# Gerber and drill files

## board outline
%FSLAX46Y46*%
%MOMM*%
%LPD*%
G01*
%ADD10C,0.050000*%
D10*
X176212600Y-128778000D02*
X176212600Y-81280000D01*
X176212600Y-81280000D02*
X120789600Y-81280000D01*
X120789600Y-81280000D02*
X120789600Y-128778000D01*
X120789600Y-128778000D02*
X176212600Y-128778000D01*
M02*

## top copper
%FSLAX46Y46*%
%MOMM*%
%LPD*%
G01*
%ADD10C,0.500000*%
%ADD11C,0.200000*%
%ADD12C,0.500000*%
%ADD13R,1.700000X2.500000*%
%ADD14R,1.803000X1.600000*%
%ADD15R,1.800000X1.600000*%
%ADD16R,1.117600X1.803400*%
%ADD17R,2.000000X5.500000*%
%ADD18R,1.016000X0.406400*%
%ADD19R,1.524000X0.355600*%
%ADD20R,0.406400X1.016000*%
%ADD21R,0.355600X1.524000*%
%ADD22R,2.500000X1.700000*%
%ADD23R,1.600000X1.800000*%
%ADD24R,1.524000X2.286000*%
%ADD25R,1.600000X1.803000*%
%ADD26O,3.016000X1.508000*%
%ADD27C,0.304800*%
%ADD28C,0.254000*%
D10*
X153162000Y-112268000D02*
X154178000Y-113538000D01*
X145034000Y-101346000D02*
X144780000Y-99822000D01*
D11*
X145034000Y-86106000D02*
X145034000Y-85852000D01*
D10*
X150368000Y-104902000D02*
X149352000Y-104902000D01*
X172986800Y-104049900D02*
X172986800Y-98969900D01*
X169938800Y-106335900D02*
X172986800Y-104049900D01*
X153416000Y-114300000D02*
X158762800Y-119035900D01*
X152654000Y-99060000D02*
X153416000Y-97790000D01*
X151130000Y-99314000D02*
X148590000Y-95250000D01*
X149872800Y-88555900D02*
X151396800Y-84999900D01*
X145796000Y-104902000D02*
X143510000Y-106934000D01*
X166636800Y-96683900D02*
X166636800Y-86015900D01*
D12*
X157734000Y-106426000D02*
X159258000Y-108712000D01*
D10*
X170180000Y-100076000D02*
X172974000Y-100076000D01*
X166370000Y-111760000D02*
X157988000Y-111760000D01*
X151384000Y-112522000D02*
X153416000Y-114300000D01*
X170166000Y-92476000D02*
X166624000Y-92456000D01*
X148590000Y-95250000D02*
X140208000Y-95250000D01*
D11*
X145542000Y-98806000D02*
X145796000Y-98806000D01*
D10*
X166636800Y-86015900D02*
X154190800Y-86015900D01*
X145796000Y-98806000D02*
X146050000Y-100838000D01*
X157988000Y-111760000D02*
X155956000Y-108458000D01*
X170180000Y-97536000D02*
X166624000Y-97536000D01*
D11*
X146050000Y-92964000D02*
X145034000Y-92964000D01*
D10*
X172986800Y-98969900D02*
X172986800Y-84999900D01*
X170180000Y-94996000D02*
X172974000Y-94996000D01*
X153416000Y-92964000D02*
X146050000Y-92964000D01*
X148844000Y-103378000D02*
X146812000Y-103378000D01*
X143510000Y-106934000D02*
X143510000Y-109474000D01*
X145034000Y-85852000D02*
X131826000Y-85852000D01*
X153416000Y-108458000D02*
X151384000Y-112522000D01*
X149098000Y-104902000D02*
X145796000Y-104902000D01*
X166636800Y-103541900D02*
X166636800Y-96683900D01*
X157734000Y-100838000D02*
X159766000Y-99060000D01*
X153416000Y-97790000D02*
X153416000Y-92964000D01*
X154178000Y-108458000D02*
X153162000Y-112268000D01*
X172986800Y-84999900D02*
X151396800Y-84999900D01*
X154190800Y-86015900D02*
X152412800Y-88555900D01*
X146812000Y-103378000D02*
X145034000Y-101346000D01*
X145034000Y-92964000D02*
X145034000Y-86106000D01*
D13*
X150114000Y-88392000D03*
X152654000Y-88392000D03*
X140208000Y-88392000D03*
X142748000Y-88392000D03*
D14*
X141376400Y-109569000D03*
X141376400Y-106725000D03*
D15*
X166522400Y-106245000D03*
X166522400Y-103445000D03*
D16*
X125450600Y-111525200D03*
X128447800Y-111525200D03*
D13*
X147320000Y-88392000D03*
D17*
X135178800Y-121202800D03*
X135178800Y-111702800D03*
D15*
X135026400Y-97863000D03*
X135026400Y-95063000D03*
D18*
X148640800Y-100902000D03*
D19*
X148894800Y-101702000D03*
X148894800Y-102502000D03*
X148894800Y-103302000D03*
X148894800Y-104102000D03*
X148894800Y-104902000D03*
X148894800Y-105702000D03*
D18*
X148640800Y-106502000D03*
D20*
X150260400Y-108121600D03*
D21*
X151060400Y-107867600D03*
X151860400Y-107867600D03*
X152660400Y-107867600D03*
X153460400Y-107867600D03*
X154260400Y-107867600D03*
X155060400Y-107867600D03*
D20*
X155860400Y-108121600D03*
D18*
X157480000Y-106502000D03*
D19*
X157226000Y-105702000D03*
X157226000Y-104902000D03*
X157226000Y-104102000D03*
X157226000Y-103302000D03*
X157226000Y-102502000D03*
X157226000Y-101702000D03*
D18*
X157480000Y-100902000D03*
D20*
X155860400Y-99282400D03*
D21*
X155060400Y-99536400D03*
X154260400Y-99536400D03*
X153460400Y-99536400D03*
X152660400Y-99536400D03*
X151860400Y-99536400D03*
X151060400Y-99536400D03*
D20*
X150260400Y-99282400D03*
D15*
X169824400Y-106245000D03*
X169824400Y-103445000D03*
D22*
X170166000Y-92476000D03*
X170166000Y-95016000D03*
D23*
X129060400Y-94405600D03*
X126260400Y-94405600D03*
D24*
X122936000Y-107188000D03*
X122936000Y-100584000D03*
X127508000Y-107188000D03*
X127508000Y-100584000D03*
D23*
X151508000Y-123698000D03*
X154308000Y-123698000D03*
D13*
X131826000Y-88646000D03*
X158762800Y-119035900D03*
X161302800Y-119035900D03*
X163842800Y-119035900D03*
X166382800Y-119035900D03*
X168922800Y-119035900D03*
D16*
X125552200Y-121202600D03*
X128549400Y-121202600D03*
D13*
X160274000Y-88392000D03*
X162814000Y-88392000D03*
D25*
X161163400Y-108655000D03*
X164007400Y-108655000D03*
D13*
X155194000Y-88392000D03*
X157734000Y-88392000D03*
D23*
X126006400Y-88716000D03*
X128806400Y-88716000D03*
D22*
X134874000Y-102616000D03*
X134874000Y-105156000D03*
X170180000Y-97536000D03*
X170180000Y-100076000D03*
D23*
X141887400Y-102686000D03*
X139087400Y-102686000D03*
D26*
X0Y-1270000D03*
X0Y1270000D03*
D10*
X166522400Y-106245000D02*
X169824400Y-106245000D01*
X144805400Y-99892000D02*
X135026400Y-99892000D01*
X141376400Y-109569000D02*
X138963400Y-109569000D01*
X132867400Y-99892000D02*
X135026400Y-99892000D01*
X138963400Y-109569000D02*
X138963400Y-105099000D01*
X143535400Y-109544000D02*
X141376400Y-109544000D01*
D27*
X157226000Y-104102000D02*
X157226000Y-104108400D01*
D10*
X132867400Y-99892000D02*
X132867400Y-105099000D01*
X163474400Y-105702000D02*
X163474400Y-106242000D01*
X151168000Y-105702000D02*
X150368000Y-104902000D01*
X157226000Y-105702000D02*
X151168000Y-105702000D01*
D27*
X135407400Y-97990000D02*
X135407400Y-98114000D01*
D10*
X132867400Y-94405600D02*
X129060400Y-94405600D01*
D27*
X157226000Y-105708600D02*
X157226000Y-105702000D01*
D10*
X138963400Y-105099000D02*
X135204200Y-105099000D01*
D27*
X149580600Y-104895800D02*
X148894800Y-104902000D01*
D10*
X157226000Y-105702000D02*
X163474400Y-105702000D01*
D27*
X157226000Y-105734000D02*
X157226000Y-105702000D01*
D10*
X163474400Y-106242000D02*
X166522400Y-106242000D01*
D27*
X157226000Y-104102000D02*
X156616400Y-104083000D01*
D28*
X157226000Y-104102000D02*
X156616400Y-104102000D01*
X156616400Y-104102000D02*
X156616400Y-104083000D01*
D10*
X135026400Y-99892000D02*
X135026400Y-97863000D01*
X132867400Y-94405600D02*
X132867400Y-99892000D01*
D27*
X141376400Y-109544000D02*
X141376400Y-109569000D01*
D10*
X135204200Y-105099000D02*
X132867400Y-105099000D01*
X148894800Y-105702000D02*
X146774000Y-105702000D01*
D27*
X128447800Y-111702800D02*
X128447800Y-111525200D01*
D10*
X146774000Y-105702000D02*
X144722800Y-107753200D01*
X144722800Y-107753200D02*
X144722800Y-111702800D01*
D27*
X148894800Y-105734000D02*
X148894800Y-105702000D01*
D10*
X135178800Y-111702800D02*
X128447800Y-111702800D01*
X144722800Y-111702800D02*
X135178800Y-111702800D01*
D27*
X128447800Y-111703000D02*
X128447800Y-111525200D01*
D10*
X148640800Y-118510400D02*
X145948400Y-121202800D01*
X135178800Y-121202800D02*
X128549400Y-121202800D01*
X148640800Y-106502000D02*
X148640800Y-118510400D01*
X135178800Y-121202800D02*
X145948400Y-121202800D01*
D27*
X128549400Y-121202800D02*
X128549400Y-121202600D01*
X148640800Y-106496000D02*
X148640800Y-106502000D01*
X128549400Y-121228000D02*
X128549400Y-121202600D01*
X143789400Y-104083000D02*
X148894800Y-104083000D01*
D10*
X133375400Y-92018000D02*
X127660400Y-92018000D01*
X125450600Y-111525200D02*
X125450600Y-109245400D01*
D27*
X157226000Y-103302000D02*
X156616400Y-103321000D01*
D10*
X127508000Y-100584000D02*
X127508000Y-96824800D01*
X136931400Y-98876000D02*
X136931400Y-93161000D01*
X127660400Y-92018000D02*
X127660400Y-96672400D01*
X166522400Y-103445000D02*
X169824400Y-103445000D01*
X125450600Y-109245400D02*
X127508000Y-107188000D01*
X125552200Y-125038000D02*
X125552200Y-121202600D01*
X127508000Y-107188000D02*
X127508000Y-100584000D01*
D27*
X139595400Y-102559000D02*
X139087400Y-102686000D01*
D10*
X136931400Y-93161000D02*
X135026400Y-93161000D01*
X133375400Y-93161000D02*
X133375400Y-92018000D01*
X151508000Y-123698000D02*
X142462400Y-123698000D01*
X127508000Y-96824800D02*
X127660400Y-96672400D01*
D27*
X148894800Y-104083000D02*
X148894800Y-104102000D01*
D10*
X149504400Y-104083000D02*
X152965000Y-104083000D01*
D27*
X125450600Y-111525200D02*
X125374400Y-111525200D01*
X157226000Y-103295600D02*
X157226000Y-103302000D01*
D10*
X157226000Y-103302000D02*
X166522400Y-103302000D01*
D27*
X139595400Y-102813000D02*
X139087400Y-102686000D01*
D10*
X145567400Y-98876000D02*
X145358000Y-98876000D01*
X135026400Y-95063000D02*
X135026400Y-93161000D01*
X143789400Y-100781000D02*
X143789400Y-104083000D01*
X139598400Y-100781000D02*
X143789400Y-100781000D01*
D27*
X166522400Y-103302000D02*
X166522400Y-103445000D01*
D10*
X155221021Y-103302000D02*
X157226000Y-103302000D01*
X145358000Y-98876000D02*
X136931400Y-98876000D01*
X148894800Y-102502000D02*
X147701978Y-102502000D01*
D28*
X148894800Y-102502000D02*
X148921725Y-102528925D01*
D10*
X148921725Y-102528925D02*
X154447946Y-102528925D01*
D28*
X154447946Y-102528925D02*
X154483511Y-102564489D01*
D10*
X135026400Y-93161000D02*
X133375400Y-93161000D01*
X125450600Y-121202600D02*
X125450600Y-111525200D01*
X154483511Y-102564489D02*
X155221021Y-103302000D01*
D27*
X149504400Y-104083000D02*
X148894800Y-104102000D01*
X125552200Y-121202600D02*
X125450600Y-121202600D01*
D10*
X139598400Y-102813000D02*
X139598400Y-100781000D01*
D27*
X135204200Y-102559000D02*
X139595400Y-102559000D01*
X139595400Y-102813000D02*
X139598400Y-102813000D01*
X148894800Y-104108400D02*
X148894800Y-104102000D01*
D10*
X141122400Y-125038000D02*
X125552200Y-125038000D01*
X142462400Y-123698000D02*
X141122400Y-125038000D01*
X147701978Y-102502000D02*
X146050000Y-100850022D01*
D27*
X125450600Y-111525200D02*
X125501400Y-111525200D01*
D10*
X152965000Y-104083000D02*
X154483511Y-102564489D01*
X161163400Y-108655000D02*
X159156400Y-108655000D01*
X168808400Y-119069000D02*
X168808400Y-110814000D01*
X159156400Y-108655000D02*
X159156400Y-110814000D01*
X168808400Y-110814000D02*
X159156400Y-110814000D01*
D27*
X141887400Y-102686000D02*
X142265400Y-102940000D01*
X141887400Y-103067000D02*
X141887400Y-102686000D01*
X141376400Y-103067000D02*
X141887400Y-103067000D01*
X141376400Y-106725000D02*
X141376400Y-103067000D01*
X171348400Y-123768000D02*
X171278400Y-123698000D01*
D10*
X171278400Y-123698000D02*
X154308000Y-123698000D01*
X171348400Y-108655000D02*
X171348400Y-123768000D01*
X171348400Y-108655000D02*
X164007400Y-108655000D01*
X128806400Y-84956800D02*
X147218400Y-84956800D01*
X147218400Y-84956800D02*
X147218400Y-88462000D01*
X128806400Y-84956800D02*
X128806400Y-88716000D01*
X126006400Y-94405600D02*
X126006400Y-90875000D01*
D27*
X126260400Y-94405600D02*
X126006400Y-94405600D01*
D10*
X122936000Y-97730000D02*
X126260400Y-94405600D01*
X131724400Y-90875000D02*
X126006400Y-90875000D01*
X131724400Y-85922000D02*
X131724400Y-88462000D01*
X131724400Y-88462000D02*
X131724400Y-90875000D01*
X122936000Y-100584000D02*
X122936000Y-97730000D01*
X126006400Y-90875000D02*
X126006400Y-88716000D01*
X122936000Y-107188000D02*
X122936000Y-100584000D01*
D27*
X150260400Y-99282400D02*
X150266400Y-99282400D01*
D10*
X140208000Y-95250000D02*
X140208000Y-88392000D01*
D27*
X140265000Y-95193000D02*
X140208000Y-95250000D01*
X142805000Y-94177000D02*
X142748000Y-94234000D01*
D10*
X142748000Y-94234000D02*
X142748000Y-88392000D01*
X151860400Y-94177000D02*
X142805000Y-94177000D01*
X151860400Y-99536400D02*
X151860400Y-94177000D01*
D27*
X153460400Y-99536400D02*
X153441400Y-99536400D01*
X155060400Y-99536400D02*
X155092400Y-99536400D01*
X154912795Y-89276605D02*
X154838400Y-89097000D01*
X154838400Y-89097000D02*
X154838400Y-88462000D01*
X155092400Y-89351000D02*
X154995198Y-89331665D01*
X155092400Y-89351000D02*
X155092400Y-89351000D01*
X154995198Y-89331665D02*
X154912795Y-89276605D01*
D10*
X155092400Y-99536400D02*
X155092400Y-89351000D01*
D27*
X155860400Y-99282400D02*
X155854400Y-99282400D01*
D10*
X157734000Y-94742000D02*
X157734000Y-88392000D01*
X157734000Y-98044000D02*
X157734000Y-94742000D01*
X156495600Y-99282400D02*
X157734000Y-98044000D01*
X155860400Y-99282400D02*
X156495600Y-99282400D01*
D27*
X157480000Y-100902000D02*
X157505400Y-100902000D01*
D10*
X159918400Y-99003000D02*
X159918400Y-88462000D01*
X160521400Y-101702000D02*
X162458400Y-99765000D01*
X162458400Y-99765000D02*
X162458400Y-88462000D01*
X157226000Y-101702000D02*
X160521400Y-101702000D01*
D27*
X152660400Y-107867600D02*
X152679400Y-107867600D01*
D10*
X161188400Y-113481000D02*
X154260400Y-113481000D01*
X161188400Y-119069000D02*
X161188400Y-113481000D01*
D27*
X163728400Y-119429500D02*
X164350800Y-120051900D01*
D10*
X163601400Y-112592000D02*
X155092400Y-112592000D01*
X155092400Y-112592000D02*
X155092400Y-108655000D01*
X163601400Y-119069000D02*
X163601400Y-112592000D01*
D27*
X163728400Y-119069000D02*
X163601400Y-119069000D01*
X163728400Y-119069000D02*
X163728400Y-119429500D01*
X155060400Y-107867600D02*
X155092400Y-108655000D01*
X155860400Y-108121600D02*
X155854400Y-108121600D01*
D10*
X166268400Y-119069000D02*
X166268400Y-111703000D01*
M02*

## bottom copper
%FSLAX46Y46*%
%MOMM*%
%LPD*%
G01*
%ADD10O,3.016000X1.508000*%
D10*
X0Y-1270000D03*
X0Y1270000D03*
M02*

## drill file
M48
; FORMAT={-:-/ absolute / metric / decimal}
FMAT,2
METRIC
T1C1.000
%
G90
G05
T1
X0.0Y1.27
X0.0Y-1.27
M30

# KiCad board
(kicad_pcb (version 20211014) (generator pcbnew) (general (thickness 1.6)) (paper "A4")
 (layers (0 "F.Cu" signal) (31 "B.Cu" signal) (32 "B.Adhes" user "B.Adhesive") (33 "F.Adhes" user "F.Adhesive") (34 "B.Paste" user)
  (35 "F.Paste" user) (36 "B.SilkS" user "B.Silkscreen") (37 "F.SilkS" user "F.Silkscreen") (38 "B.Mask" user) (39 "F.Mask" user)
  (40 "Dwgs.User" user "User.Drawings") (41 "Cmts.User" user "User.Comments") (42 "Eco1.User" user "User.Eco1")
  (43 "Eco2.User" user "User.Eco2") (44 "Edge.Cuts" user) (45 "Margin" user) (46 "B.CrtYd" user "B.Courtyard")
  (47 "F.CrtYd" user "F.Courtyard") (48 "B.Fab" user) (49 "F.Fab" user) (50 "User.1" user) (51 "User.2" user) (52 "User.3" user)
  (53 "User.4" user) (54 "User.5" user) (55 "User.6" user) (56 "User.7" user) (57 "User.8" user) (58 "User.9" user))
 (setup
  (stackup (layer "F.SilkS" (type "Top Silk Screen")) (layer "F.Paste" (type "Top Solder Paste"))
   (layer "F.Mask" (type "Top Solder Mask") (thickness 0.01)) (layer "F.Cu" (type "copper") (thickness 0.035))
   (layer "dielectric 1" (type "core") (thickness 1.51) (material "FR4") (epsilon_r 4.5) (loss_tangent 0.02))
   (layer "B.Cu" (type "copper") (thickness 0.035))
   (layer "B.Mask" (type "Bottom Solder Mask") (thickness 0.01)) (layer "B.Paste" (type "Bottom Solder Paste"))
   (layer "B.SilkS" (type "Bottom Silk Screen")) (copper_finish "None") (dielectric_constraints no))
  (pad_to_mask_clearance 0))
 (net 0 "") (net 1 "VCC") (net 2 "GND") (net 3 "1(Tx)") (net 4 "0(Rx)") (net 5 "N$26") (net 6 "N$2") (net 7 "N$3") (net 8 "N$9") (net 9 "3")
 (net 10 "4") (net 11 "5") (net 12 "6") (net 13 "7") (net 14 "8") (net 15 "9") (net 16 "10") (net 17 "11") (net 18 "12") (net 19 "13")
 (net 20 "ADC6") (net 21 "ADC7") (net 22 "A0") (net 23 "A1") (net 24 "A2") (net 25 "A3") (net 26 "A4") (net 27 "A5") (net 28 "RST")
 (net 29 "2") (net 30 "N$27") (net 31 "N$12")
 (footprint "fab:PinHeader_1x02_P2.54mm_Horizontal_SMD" (layer "F.Cu") (at 150.114 88.392 90)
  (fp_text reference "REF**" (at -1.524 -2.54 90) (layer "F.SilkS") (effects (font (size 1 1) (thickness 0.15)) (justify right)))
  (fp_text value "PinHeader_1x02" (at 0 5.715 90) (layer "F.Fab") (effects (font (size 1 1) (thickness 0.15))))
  (pad "1" smd rect locked (at 0 0 90) (size 2.5 1.7) (layers "F.Cu" "F.Paste" "F.Mask") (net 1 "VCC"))
  (pad "2" smd rect locked (at 0 2.54 90) (size 2.5 1.7) (layers "F.Cu" "F.Paste" "F.Mask") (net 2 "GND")))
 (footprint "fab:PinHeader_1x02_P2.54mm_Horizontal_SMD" (layer "F.Cu") (at 140.208 88.392 90)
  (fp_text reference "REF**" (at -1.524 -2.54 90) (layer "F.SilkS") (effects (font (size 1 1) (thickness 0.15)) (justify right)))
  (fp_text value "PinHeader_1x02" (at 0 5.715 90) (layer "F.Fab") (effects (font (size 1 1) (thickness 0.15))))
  (pad "1" smd rect locked (at 0 0 90) (size 2.5 1.7) (layers "F.Cu" "F.Paste" "F.Mask") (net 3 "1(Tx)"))
  (pad "2" smd rect locked (at 0 2.54 90) (size 2.5 1.7) (layers "F.Cu" "F.Paste" "F.Mask") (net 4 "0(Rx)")))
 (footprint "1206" (layer "F.Cu") (at 141.3764 108.147 90)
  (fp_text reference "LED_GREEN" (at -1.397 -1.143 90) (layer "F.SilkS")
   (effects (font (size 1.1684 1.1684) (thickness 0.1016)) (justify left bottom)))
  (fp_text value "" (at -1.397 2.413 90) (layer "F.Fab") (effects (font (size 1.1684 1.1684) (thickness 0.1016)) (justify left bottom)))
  (pad "1" smd rect (at -1.422 0 90) (size 1.6 1.803) (layers "F.Cu" "F.Paste" "F.Mask") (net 1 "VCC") (solder_mask_margin 0.1016))
  (pad "2" smd rect (at 1.422 0 90) (size 1.6 1.803) (layers "F.Cu" "F.Paste" "F.Mask") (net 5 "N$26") (solder_mask_margin 0.1016)))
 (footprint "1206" (layer "F.Cu") (at 166.5224 104.845 90)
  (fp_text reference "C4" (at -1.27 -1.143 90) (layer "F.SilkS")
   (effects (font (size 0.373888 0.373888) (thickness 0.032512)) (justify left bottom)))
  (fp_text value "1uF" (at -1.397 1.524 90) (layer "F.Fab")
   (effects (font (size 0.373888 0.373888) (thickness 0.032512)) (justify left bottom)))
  (pad "1" smd rect (at -1.4 0 90) (size 1.6 1.8) (layers "F.Cu" "F.Paste" "F.Mask") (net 1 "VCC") (solder_mask_margin 0.1016))
  (pad "2" smd rect (at 1.4 0 90) (size 1.6 1.8) (layers "F.Cu" "F.Paste" "F.Mask") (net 2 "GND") (solder_mask_margin 0.1016)))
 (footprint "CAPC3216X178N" (layer "F.Cu") (at 126.9492 111.5252)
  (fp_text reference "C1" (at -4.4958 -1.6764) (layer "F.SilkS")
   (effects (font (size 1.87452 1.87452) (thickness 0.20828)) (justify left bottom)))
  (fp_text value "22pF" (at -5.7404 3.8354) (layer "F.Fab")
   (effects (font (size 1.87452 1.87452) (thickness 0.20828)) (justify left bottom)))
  (pad "1" smd rect (at -1.4986 0) (size 1.1176 1.8034) (layers "F.Cu" "F.Paste" "F.Mask") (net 2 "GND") (solder_mask_margin 0.1016))
  (pad "2" smd rect (at 1.4986 0) (size 1.1176 1.8034) (layers "F.Cu" "F.Paste" "F.Mask") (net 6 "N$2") (solder_mask_margin 0.1016)))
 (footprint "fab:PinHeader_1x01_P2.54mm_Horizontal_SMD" (layer "F.Cu") (at 147.32 88.392 90)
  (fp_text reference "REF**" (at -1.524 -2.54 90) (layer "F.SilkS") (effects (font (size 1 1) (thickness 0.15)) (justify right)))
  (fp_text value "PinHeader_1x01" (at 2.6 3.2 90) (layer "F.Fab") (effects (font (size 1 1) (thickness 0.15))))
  (pad "1" smd rect locked (at 0 0 90) (size 2.5 1.7) (layers "F.Cu" "F.Paste" "F.Mask") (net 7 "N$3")))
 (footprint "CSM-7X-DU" (layer "F.Cu") (at 135.1788 116.4528 90)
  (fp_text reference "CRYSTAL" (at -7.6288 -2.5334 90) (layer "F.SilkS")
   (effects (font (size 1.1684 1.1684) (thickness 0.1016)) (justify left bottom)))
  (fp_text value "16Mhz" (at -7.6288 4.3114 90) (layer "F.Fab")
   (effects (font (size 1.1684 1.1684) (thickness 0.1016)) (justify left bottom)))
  (pad "1" smd rect (at -4.75 0 90) (size 5.5 2) (layers "F.Cu" "F.Paste" "F.Mask") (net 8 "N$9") (solder_mask_margin 0.1016))
  (pad "2" smd rect (at 4.75 0 90) (size 5.5 2) (layers "F.Cu" "F.Paste" "F.Mask") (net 6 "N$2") (solder_mask_margin 0.1016)))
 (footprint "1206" (layer "F.Cu") (at 135.0264 96.463 90)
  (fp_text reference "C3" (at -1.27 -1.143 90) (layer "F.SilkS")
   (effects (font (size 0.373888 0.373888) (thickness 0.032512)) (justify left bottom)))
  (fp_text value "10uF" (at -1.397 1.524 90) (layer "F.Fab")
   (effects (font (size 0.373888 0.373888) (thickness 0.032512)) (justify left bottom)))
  (pad "1" smd rect (at -1.4 0 90) (size 1.6 1.8) (layers "F.Cu" "F.Paste" "F.Mask") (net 1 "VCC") (solder_mask_margin 0.1016))
  (pad "2" smd rect (at 1.4 0 90) (size 1.6 1.8) (layers "F.Cu" "F.Paste" "F.Mask") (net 2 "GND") (solder_mask_margin 0.1016)))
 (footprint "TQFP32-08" (layer "F.Cu") (at 153.0604 103.702)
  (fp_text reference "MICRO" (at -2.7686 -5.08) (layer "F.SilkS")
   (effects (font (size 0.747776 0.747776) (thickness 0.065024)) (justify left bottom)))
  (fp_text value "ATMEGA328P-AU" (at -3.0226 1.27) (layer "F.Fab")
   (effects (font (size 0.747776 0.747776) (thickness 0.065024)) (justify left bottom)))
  (pad "1" smd rect (at -4.4196 -2.8) (size 1.016 0.4064) (layers "F.Cu" "F.Paste" "F.Mask") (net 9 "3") (solder_mask_margin 0.1016))
  (pad "2" smd rect (at -4.1656 -2) (size 1.524 0.3556) (layers "F.Cu" "F.Paste" "F.Mask") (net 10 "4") (solder_mask_margin 0.1016))
  (pad "3" smd rect (at -4.1656 -1.2) (size 1.524 0.3556) (layers "F.Cu" "F.Paste" "F.Mask") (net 2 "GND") (solder_mask_margin 0.1016))
  (pad "4" smd rect (at -4.1656 -0.4) (size 1.524 0.3556) (layers "F.Cu" "F.Paste" "F.Mask") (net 1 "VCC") (solder_mask_margin 0.1016))
  (pad "5" smd rect (at -4.1656 0.4) (size 1.524 0.3556) (layers "F.Cu" "F.Paste" "F.Mask") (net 2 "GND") (solder_mask_margin 0.1016))
  (pad "6" smd rect (at -4.1656 1.2) (size 1.524 0.3556) (layers "F.Cu" "F.Paste" "F.Mask") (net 1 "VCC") (solder_mask_margin 0.1016))
  (pad "7" smd rect (at -4.1656 2) (size 1.524 0.3556) (layers "F.Cu" "F.Paste" "F.Mask") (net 6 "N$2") (solder_mask_margin 0.1016))
  (pad "8" smd rect (at -4.4196 2.8) (size 1.016 0.4064) (layers "F.Cu" "F.Paste" "F.Mask") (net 8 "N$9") (solder_mask_margin 0.1016))
  (pad "9" smd rect (at -2.8 4.4196) (size 0.4064 1.016) (layers "F.Cu" "F.Paste" "F.Mask") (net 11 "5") (solder_mask_margin 0.1016))
  (pad "10" smd rect (at -2 4.1656) (size 0.3556 1.524) (layers "F.Cu" "F.Paste" "F.Mask") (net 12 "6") (solder_mask_margin 0.1016))
  (pad "11" smd rect (at -1.2 4.1656) (size 0.3556 1.524) (layers "F.Cu" "F.Paste" "F.Mask") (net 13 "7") (solder_mask_margin 0.1016))
  (pad "12" smd rect (at -0.4 4.1656) (size 0.3556 1.524) (layers "F.Cu" "F.Paste" "F.Mask") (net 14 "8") (solder_mask_margin 0.1016))
  (pad "13" smd rect (at 0.4 4.1656) (size 0.3556 1.524) (layers "F.Cu" "F.Paste" "F.Mask") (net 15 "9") (solder_mask_margin 0.1016))
  (pad "14" smd rect (at 1.2 4.1656) (size 0.3556 1.524) (layers "F.Cu" "F.Paste" "F.Mask") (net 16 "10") (solder_mask_margin 0.1016))
  (pad "15" smd rect (at 2 4.1656) (size 0.3556 1.524) (layers "F.Cu" "F.Paste" "F.Mask") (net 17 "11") (solder_mask_margin 0.1016))
  (pad "16" smd rect (at 2.8 4.4196) (size 0.4064 1.016) (layers "F.Cu" "F.Paste" "F.Mask") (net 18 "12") (solder_mask_margin 0.1016))
  (pad "17" smd rect (at 4.4196 2.8) (size 1.016 0.4064) (layers "F.Cu" "F.Paste" "F.Mask") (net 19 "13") (solder_mask_margin 0.1016))
  (pad "18" smd rect (at 4.1656 2) (size 1.524 0.3556) (layers "F.Cu" "F.Paste" "F.Mask") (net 1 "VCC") (solder_mask_margin 0.1016))
  (pad "19" smd rect (at 4.1656 1.2) (size 1.524 0.3556) (layers "F.Cu" "F.Paste" "F.Mask") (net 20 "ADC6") (solder_mask_margin 0.1016))
  (pad "20" smd rect (at 4.1656 0.4) (size 1.524 0.3556) (layers "F.Cu" "F.Paste" "F.Mask") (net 1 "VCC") (solder_mask_margin 0.1016))
  (pad "21" smd rect (at 4.1656 -0.4) (size 1.524 0.3556) (layers "F.Cu" "F.Paste" "F.Mask") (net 2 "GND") (solder_mask_margin 0.1016))
  (pad "22" smd rect (at 4.1656 -1.2) (size 1.524 0.3556) (layers "F.Cu" "F.Paste" "F.Mask") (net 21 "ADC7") (solder_mask_margin 0.1016))
  (pad "23" smd rect (at 4.1656 -2) (size 1.524 0.3556) (layers "F.Cu" "F.Paste" "F.Mask") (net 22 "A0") (solder_mask_margin 0.1016))
  (pad "24" smd rect (at 4.4196 -2.8) (size 1.016 0.4064) (layers "F.Cu" "F.Paste" "F.Mask") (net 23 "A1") (solder_mask_margin 0.1016))
  (pad "25" smd rect (at 2.8 -4.4196) (size 0.4064 1.016) (layers "F.Cu" "F.Paste" "F.Mask") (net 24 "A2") (solder_mask_margin 0.1016))
  (pad "26" smd rect (at 2 -4.1656) (size 0.3556 1.524) (layers "F.Cu" "F.Paste" "F.Mask") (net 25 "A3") (solder_mask_margin 0.1016))
  (pad "27" smd rect (at 1.2 -4.1656) (size 0.3556 1.524) (layers "F.Cu" "F.Paste" "F.Mask") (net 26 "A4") (solder_mask_margin 0.1016))
  (pad "28" smd rect (at 0.4 -4.1656) (size 0.3556 1.524) (layers "F.Cu" "F.Paste" "F.Mask") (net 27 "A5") (solder_mask_margin 0.1016))
  (pad "29" smd rect (at -0.4 -4.1656) (size 0.3556 1.524) (layers "F.Cu" "F.Paste" "F.Mask") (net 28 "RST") (solder_mask_margin 0.1016))
  (pad "30" smd rect (at -1.2 -4.1656) (size 0.3556 1.524) (layers "F.Cu" "F.Paste" "F.Mask") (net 4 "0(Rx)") (solder_mask_margin 0.1016))
  (pad "31" smd rect (at -2 -4.1656) (size 0.3556 1.524) (layers "F.Cu" "F.Paste" "F.Mask") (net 3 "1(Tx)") (solder_mask_margin 0.1016))
  (pad "32" smd rect (at -2.8 -4.4196) (size 0.4064 1.016) (layers "F.Cu" "F.Paste" "F.Mask") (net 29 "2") (solder_mask_margin 0.1016)))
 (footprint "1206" (layer "F.Cu") (at 169.8244 104.845 90)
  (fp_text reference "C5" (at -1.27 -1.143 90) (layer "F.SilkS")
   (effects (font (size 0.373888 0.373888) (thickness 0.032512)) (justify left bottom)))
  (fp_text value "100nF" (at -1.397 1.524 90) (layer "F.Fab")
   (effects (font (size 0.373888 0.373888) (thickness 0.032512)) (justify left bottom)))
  (pad "1" smd rect (at -1.4 0 90) (size 1.6 1.8) (layers "F.Cu" "F.Paste" "F.Mask") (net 1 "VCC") (solder_mask_margin 0.1016))
  (pad "2" smd rect (at 1.4 0 90) (size 1.6 1.8) (layers "F.Cu" "F.Paste" "F.Mask") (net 2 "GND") (solder_mask_margin 0.1016)))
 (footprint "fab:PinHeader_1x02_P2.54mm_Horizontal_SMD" (layer "F.Cu") (at 170.166 92.476)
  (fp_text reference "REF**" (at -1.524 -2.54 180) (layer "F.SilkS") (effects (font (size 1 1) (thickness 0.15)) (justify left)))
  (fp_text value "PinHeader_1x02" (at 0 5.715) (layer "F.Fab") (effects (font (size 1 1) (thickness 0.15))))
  (pad "1" smd rect locked (at 0 0) (size 2.5 1.7) (layers "F.Cu" "F.Paste" "F.Mask") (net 2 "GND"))
  (pad "2" smd rect locked (at 0 2.54) (size 2.5 1.7) (layers "F.Cu" "F.Paste" "F.Mask") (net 1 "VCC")))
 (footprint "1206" (layer "F.Cu") (at 127.6604 94.4056 180)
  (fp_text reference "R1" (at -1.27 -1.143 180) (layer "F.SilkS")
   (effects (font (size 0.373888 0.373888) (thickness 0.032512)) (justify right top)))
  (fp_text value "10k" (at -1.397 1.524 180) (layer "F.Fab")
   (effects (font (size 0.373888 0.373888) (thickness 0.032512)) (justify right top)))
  (pad "1" smd rect (at -1.4 0 180) (size 1.6 1.8) (layers "F.Cu" "F.Paste" "F.Mask") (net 1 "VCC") (solder_mask_margin 0.1016))
  (pad "2" smd rect (at 1.4 0 180) (size 1.6 1.8) (layers "F.Cu" "F.Paste" "F.Mask") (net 28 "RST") (solder_mask_margin 0.1016)))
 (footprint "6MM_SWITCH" (layer "F.Cu") (at 125.222 103.886 90)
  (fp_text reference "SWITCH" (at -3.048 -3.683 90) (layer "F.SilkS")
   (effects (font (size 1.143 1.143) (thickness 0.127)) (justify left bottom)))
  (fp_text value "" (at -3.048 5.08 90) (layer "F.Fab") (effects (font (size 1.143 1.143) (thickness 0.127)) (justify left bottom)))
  (pad "1" smd rect (at -3.302 -2.286 90) (size 2.286 1.524) (layers "F.Cu" "F.Paste" "F.Mask") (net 28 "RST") (solder_mask_margin 0.1016))
  (pad "2" smd rect (at 3.302 -2.286 90) (size 2.286 1.524) (layers "F.Cu" "F.Paste" "F.Mask") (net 28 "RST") (solder_mask_margin 0.1016))
  (pad "3" smd rect (at -3.302 2.286 90) (size 2.286 1.524) (layers "F.Cu" "F.Paste" "F.Mask") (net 2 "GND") (solder_mask_margin 0.1016))
  (pad "4" smd rect (at 3.302 2.286 90) (size 2.286 1.524) (layers "F.Cu" "F.Paste" "F.Mask") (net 2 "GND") (solder_mask_margin 0.1016)))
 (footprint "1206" (layer "F.Cu") (at 152.908 123.698)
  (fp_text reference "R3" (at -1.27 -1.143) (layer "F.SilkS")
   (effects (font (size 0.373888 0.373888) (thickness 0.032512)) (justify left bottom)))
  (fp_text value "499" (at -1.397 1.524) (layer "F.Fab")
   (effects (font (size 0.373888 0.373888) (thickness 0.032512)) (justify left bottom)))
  (pad "1" smd rect (at -1.4 0) (size 1.6 1.8) (layers "F.Cu" "F.Paste" "F.Mask") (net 2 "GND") (solder_mask_margin 0.1016))
  (pad "2" smd rect (at 1.4 0) (size 1.6 1.8) (layers "F.Cu" "F.Paste" "F.Mask") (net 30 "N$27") (solder_mask_margin 0.1016)))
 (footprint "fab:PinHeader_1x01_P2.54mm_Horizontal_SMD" (layer "F.Cu") (at 131.826 88.646 90)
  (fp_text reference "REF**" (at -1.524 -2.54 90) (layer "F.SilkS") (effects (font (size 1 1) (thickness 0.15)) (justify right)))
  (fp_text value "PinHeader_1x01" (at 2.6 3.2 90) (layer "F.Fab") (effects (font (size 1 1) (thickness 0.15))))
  (pad "1" smd rect locked (at 0 0 90) (size 2.5 1.7) (layers "F.Cu" "F.Paste" "F.Mask") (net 28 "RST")))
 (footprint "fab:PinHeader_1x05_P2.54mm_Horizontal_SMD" (layer "F.Cu") (at 158.7628 119.0359 90)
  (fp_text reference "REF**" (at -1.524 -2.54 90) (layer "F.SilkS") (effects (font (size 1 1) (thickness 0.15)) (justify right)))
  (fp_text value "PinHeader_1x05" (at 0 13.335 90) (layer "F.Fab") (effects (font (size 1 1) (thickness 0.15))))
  (pad "1" smd rect locked (at 0 0 90) (size 2.5 1.7) (layers "F.Cu" "F.Paste" "F.Mask"))
  (pad "2" smd rect locked (at 0 2.54 90) (size 2.5 1.7) (layers "F.Cu" "F.Paste" "F.Mask") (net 16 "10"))
  (pad "3" smd rect locked (at 0 5.08 90) (size 2.5 1.7) (layers "F.Cu" "F.Paste" "F.Mask") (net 17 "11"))
  (pad "4" smd rect locked (at 0 7.62 90) (size 2.5 1.7) (layers "F.Cu" "F.Paste" "F.Mask") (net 18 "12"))
  (pad "5" smd rect locked (at 0 10.16 90) (size 2.5 1.7) (layers "F.Cu" "F.Paste" "F.Mask") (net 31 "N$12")))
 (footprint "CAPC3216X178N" (layer "F.Cu") (at 127.0508 121.2026)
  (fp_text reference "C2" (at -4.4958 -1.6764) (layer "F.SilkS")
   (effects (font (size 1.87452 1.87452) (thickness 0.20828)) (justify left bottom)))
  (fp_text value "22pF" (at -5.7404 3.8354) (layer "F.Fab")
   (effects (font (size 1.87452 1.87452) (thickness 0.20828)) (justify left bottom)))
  (pad "1" smd rect (at -1.4986 0) (size 1.1176 1.8034) (layers "F.Cu" "F.Paste" "F.Mask") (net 2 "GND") (solder_mask_margin 0.1016))
  (pad "2" smd rect (at 1.4986 0) (size 1.1176 1.8034) (layers "F.Cu" "F.Paste" "F.Mask") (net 8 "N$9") (solder_mask_margin 0.1016)))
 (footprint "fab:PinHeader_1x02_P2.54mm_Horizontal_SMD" (layer "F.Cu") (at 160.274 88.392 90)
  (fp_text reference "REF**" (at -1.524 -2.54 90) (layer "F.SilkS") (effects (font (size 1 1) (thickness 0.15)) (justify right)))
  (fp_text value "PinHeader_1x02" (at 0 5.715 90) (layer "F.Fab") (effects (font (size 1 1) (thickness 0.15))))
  (pad "1" smd rect locked (at 0 0 90) (size 2.5 1.7) (layers "F.Cu" "F.Paste" "F.Mask") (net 23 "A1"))
  (pad "2" smd rect locked (at 0 2.54 90) (size 2.5 1.7) (layers "F.Cu" "F.Paste" "F.Mask") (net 22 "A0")))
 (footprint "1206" (layer "F.Cu") (at 162.5854 108.655)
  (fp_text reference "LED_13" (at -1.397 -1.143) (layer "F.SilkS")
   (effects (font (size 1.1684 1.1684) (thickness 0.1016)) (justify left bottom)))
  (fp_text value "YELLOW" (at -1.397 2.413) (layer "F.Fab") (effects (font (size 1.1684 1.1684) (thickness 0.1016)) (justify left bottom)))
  (pad "1" smd rect (at -1.422 0) (size 1.6 1.803) (layers "F.Cu" "F.Paste" "F.Mask") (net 31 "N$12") (solder_mask_margin 0.1016))
  (pad "2" smd rect (at 1.422 0) (size 1.6 1.803) (layers "F.Cu" "F.Paste" "F.Mask") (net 30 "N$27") (solder_mask_margin 0.1016)))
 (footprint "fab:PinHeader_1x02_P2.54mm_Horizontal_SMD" (layer "F.Cu") (at 155.194 88.392 90)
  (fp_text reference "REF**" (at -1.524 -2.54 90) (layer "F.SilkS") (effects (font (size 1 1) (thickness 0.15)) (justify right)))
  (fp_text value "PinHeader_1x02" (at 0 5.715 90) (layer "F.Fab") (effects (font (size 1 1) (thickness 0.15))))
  (pad "1" smd rect locked (at 0 0 90) (size 2.5 1.7) (layers "F.Cu" "F.Paste" "F.Mask") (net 25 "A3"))
  (pad "2" smd rect locked (at 0 2.54 90) (size 2.5 1.7) (layers "F.Cu" "F.Paste" "F.Mask") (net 24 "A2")))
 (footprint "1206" (layer "F.Cu") (at 127.4064 88.716)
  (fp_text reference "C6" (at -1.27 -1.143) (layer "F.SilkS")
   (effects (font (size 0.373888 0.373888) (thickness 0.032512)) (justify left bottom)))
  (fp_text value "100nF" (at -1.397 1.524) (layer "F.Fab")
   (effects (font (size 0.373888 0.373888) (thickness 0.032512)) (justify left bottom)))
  (pad "1" smd rect (at -1.4 0) (size 1.6 1.8) (layers "F.Cu" "F.Paste" "F.Mask") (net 28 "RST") (solder_mask_margin 0.1016))
  (pad "2" smd rect (at 1.4 0) (size 1.6 1.8) (layers "F.Cu" "F.Paste" "F.Mask") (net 7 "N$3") (solder_mask_margin 0.1016)))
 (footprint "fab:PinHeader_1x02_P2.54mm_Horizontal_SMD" (layer "F.Cu") (at 134.874 102.616)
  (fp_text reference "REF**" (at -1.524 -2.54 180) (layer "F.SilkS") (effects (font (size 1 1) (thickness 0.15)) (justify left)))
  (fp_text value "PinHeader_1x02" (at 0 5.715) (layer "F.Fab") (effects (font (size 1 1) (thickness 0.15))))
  (pad "1" smd rect locked (at 0 0) (size 2.5 1.7) (layers "F.Cu" "F.Paste" "F.Mask") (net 2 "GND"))
  (pad "2" smd rect locked (at 0 2.54) (size 2.5 1.7) (layers "F.Cu" "F.Paste" "F.Mask") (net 1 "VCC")))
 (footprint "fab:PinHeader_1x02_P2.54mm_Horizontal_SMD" (layer "F.Cu") (at 170.18 97.536)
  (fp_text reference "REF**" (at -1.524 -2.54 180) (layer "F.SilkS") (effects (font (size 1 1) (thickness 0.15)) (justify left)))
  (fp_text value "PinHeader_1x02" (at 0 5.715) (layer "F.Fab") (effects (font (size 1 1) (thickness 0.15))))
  (pad "1" smd rect locked (at 0 0) (size 2.5 1.7) (layers "F.Cu" "F.Paste" "F.Mask") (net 2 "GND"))
  (pad "2" smd rect locked (at 0 2.54) (size 2.5 1.7) (layers "F.Cu" "F.Paste" "F.Mask") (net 1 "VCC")))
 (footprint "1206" (layer "F.Cu") (at 140.4874 102.686 180)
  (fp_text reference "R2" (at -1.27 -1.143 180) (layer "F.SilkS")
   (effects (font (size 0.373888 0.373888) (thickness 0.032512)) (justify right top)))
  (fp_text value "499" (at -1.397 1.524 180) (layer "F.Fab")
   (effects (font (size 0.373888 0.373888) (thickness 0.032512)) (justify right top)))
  (pad "1" smd rect (at -1.4 0 180) (size 1.6 1.8) (layers "F.Cu" "F.Paste" "F.Mask") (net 5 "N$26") (solder_mask_margin 0.1016))
  (pad "2" smd rect (at 1.4 0 180) (size 1.6 1.8) (layers "F.Cu" "F.Paste" "F.Mask") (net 2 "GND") (solder_mask_margin 0.1016)))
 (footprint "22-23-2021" (layer "F.Cu") (at 0 0 90)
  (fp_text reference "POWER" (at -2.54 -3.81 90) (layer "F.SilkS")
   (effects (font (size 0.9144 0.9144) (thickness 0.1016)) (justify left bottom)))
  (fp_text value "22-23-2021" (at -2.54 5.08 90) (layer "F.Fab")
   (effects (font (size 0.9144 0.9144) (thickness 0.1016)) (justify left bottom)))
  (pad "1" thru_hole oval (at -1.27 0 180) (size 3.016 1.508) (drill 1) (layers *.Cu *.Mask) (solder_mask_margin 0.1016))
  (pad "2" thru_hole oval (at 1.27 0 180) (size 3.016 1.508) (drill 1) (layers *.Cu *.Mask) (solder_mask_margin 0.1016)))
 (gr_line (start 153.162 112.268) (end 154.178 113.538) (layer "F.Cu") (width 0.5))
 (gr_line (start 145.034 101.346) (end 144.78 99.822) (layer "F.Cu") (width 0.5))
 (gr_line (start 145.034 86.106) (end 145.034 85.852) (layer "F.Cu") (width 0.2))
 (gr_line (start 150.368 104.902) (end 149.352 104.902) (layer "F.Cu") (width 0.5))
 (gr_line (start 172.9868 104.0499) (end 172.9868 98.9699) (layer "F.Cu") (width 0.5))
 (gr_line (start 169.9388 106.3359) (end 172.9868 104.0499) (layer "F.Cu") (width 0.5))
 (gr_line (start 153.416 114.3) (end 158.7628 119.0359) (layer "F.Cu") (width 0.5))
 (gr_line (start 152.654 99.06) (end 153.416 97.79) (layer "F.Cu") (width 0.5))
 (gr_line (start 151.13 99.314) (end 148.59 95.25) (layer "F.Cu") (width 0.5))
 (gr_line (start 149.8728 88.5559) (end 151.3968 84.9999) (layer "F.Cu") (width 0.5))
 (gr_line (start 145.796 104.902) (end 143.51 106.934) (layer "F.Cu") (width 0.5))
 (gr_line (start 166.6368 96.6839) (end 166.6368 86.0159) (layer "F.Cu") (width 0.5))
 (gr_line (start 157.734 106.426) (end 159.258 108.712) (layer "F.Cu") (width 0.5))
 (gr_line (start 170.18 100.076) (end 172.974 100.076) (layer "F.Cu") (width 0.5))
 (gr_line (start 166.37 111.76) (end 157.988 111.76) (layer "F.Cu") (width 0.5))
 (gr_line (start 151.384 112.522) (end 153.416 114.3) (layer "F.Cu") (width 0.5))
 (gr_line (start 170.166 92.476) (end 166.624 92.456) (layer "F.Cu") (width 0.5))
 (gr_line (start 148.59 95.25) (end 140.208 95.25) (layer "F.Cu") (width 0.5))
 (gr_line (start 145.542 98.806) (end 145.796 98.806) (layer "F.Cu") (width 0.2))
 (gr_line (start 166.6368 86.0159) (end 154.1908 86.0159) (layer "F.Cu") (width 0.5))
 (gr_line (start 145.796 98.806) (end 146.05 100.838) (layer "F.Cu") (width 0.5))
 (gr_line (start 157.988 111.76) (end 155.956 108.458) (layer "F.Cu") (width 0.5))
 (gr_line (start 170.18 97.536) (end 166.624 97.536) (layer "F.Cu") (width 0.5))
 (gr_line (start 146.05 92.964) (end 145.034 92.964) (layer "F.Cu") (width 0.2))
 (gr_line (start 172.9868 98.9699) (end 172.9868 84.9999) (layer "F.Cu") (width 0.5))
 (gr_line (start 170.18 94.996) (end 172.974 94.996) (layer "F.Cu") (width 0.5))
 (gr_line (start 153.416 92.964) (end 146.05 92.964) (layer "F.Cu") (width 0.5))
 (gr_line (start 148.844 103.378) (end 146.812 103.378) (layer "F.Cu") (width 0.5))
 (gr_line (start 143.51 106.934) (end 143.51 109.474) (layer "F.Cu") (width 0.5))
 (gr_line (start 145.034 85.852) (end 131.826 85.852) (layer "F.Cu") (width 0.5))
 (gr_line (start 153.416 108.458) (end 151.384 112.522) (layer "F.Cu") (width 0.5))
 (gr_line (start 149.098 104.902) (end 145.796 104.902) (layer "F.Cu") (width 0.5))
 (gr_line (start 166.6368 103.5419) (end 166.6368 96.6839) (layer "F.Cu") (width 0.5))
 (gr_line (start 157.734 100.838) (end 159.766 99.06) (layer "F.Cu") (width 0.5))
 (gr_line (start 153.416 97.79) (end 153.416 92.964) (layer "F.Cu") (width 0.5))
 (gr_line (start 154.178 108.458) (end 153.162 112.268) (layer "F.Cu") (width 0.5))
 (gr_line (start 172.9868 84.9999) (end 151.3968 84.9999) (layer "F.Cu") (width 0.5))
 (gr_line (start 154.1908 86.0159) (end 152.4128 88.5559) (layer "F.Cu") (width 0.5))
 (gr_line (start 146.812 103.378) (end 145.034 101.346) (layer "F.Cu") (width 0.5))
 (gr_line (start 145.034 92.964) (end 145.034 86.106) (layer "F.Cu") (width 0.5))
 (gr_line (start 176.2126 128.778) (end 176.2126 81.28) (layer "Edge.Cuts") (width 0.05))
 (gr_line (start 176.2126 81.28) (end 120.7896 81.28) (layer "Edge.Cuts") (width 0.05))
 (gr_line (start 120.7896 81.28) (end 120.7896 128.778) (layer "Edge.Cuts") (width 0.05))
 (gr_line (start 120.7896 128.778) (end 176.2126 128.778) (layer "Edge.Cuts") (width 0.05))
 (segment (start 166.5224 106.245) (end 169.8244 106.245) (width 0.5) (layer "F.Cu") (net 1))
 (segment (start 144.8054 99.892) (end 135.0264 99.892) (width 0.5) (layer "F.Cu") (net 1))
 (segment (start 141.3764 109.569) (end 138.9634 109.569) (width 0.5) (layer "F.Cu") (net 1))
 (segment (start 132.8674 99.892) (end 135.0264 99.892) (width 0.5) (layer "F.Cu") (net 1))
 (segment (start 138.9634 109.569) (end 138.9634 105.099) (width 0.5) (layer "F.Cu") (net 1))
 (segment (start 143.5354 109.544) (end 141.3764 109.544) (width 0.5) (layer "F.Cu") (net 1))
 (segment (start 157.226 104.102) (end 157.226 104.1084) (width 0.3048) (layer "F.Cu") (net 1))
 (segment (start 132.8674 99.892) (end 132.8674 105.099) (width 0.5) (layer "F.Cu") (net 1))
 (segment (start 163.4744 105.702) (end 163.4744 106.242) (width 0.5) (layer "F.Cu") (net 1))
 (segment (start 151.168 105.702) (end 150.368 104.902) (width 0.5) (layer "F.Cu") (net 1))
 (segment (start 157.226 105.702) (end 151.168 105.702) (width 0.5) (layer "F.Cu") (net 1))
 (segment (start 135.4074 97.99) (end 135.4074 98.114) (width 0.3048) (layer "F.Cu") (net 1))
 (segment (start 132.8674 94.4056) (end 129.0604 94.4056) (width 0.5) (layer "F.Cu") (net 1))
 (segment (start 157.226 105.7086) (end 157.226 105.702) (width 0.3048) (layer "F.Cu") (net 1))
 (segment (start 138.9634 105.099) (end 135.2042 105.099) (width 0.5) (layer "F.Cu") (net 1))
 (segment (start 149.5806 104.8958) (end 148.8948 104.902) (width 0.3048) (layer "F.Cu") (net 1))
 (segment (start 157.226 105.702) (end 163.4744 105.702) (width 0.5) (layer "F.Cu") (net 1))
 (segment (start 157.226 105.734) (end 157.226 105.702) (width 0.3048) (layer "F.Cu") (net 1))
 (segment (start 163.4744 106.242) (end 166.5224 106.242) (width 0.5) (layer "F.Cu") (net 1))
 (segment (start 157.226 104.102) (end 156.6164 104.083) (width 0.3048) (layer "F.Cu") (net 1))
 (segment (start 157.226 104.102) (end 156.6164 104.102) (width 0.254) (layer "F.Cu") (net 1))
 (segment (start 156.6164 104.102) (end 156.6164 104.083) (width 0.254) (layer "F.Cu") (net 1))
 (segment (start 135.0264 99.892) (end 135.0264 97.863) (width 0.5) (layer "F.Cu") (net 1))
 (segment (start 132.8674 94.4056) (end 132.8674 99.892) (width 0.5) (layer "F.Cu") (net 1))
 (segment (start 141.3764 109.544) (end 141.3764 109.569) (width 0.3048) (layer "F.Cu") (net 1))
 (segment (start 135.2042 105.099) (end 132.8674 105.099) (width 0.5) (layer "F.Cu") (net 1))
 (segment (start 148.8948 105.702) (end 146.774 105.702) (width 0.5) (layer "F.Cu") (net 6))
 (segment (start 128.4478 111.7028) (end 128.4478 111.5252) (width 0.3048) (layer "F.Cu") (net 6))
 (segment (start 146.774 105.702) (end 144.7228 107.7532) (width 0.5) (layer "F.Cu") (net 6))
 (segment (start 144.7228 107.7532) (end 144.7228 111.7028) (width 0.5) (layer "F.Cu") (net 6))
 (segment (start 148.8948 105.734) (end 148.8948 105.702) (width 0.3048) (layer "F.Cu") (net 6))
 (segment (start 135.1788 111.7028) (end 128.4478 111.7028) (width 0.5) (layer "F.Cu") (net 6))
 (segment (start 144.7228 111.7028) (end 135.1788 111.7028) (width 0.5) (layer "F.Cu") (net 6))
 (segment (start 128.4478 111.703) (end 128.4478 111.5252) (width 0.3048) (layer "F.Cu") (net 6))
 (segment (start 148.6408 118.5104) (end 145.9484 121.2028) (width 0.5) (layer "F.Cu") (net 8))
 (segment (start 135.1788 121.2028) (end 128.5494 121.2028) (width 0.5) (layer "F.Cu") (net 8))
 (segment (start 148.6408 106.502) (end 148.6408 118.5104) (width 0.5) (layer "F.Cu") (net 8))
 (segment (start 135.1788 121.2028) (end 145.9484 121.2028) (width 0.5) (layer "F.Cu") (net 8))
 (segment (start 128.5494 121.2028) (end 128.5494 121.2026) (width 0.3048) (layer "F.Cu") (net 8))
 (segment (start 148.6408 106.496) (end 148.6408 106.502) (width 0.3048) (layer "F.Cu") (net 8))
 (segment (start 128.5494 121.228) (end 128.5494 121.2026) (width 0.3048) (layer "F.Cu") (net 8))
 (segment (start 143.7894 104.083) (end 148.8948 104.083) (width 0.3048) (layer "F.Cu") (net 2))
 (segment (start 133.3754 92.018) (end 127.6604 92.018) (width 0.5) (layer "F.Cu") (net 2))
 (segment (start 125.4506 111.5252) (end 125.4506 109.2454) (width 0.5) (layer "F.Cu") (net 2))
 (segment (start 157.226 103.302) (end 156.6164 103.321) (width 0.3048) (layer "F.Cu") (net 2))
 (segment (start 127.508 100.584) (end 127.508 96.8248) (width 0.5) (layer "F.Cu") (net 2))
 (segment (start 136.9314 98.876) (end 136.9314 93.161) (width 0.5) (layer "F.Cu") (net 2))
 (segment (start 127.6604 92.018) (end 127.6604 96.6724) (width 0.5) (layer "F.Cu") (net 2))
 (segment (start 166.5224 103.445) (end 169.8244 103.445) (width 0.5) (layer "F.Cu") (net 2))
 (segment (start 125.4506 109.2454) (end 127.508 107.188) (width 0.5) (layer "F.Cu") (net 2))
 (segment (start 125.5522 125.038) (end 125.5522 121.2026) (width 0.5) (layer "F.Cu") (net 2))
 (segment (start 127.508 107.188) (end 127.508 100.584) (width 0.5) (layer "F.Cu") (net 2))
 (segment (start 139.5954 102.559) (end 139.0874 102.686) (width 0.3048) (layer "F.Cu") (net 2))
 (segment (start 136.9314 93.161) (end 135.0264 93.161) (width 0.5) (layer "F.Cu") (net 2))
 (segment (start 133.3754 93.161) (end 133.3754 92.018) (width 0.5) (layer "F.Cu") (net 2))
 (segment (start 151.508 123.698) (end 142.4624 123.698) (width 0.5) (layer "F.Cu") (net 2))
 (segment (start 127.508 96.8248) (end 127.6604 96.6724) (width 0.5) (layer "F.Cu") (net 2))
 (segment (start 148.8948 104.083) (end 148.8948 104.102) (width 0.3048) (layer "F.Cu") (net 2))
 (segment (start 149.5044 104.083) (end 152.965 104.083) (width 0.5) (layer "F.Cu") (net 2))
 (segment (start 125.4506 111.5252) (end 125.3744 111.5252) (width 0.3048) (layer "F.Cu") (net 2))
 (segment (start 157.226 103.2956) (end 157.226 103.302) (width 0.3048) (layer "F.Cu") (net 2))
 (segment (start 157.226 103.302) (end 166.5224 103.302) (width 0.5) (layer "F.Cu") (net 2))
 (segment (start 139.5954 102.813) (end 139.0874 102.686) (width 0.3048) (layer "F.Cu") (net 2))
 (segment (start 145.5674 98.876) (end 145.358 98.876) (width 0.5) (layer "F.Cu") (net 2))
 (segment (start 135.0264 95.063) (end 135.0264 93.161) (width 0.5) (layer "F.Cu") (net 2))
 (segment (start 143.7894 100.781) (end 143.7894 104.083) (width 0.5) (layer "F.Cu") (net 2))
 (segment (start 139.5984 100.781) (end 143.7894 100.781) (width 0.5) (layer "F.Cu") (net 2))
 (segment (start 166.5224 103.302) (end 166.5224 103.445) (width 0.3048) (layer "F.Cu") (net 2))
 (segment (start 155.221021 103.302) (end 157.226 103.302) (width 0.5) (layer "F.Cu") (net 2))
 (segment (start 145.358 98.876) (end 136.9314 98.876) (width 0.5) (layer "F.Cu") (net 2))
 (segment (start 148.8948 102.502) (end 147.701978 102.502) (width 0.5) (layer "F.Cu") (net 2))
 (segment (start 148.8948 102.502) (end 148.921725 102.528925) (width 0.254) (layer "F.Cu") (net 2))
 (segment (start 148.921725 102.528925) (end 154.447946 102.528925) (width 0.5) (layer "F.Cu") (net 2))
 (segment (start 154.447946 102.528925) (end 154.483511 102.564489) (width 0.254) (layer "F.Cu") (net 2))
 (segment (start 135.0264 93.161) (end 133.3754 93.161) (width 0.5) (layer "F.Cu") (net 2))
 (segment (start 125.4506 121.2026) (end 125.4506 111.5252) (width 0.5) (layer "F.Cu") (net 2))
 (segment (start 154.483511 102.564489) (end 155.221021 103.302) (width 0.5) (layer "F.Cu") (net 2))
 (segment (start 149.5044 104.083) (end 148.8948 104.102) (width 0.3048) (layer "F.Cu") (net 2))
 (segment (start 125.5522 121.2026) (end 125.4506 121.2026) (width 0.3048) (layer "F.Cu") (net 2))
 (segment (start 139.5984 102.813) (end 139.5984 100.781) (width 0.5) (layer "F.Cu") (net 2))
 (segment (start 135.2042 102.559) (end 139.5954 102.559) (width 0.3048) (layer "F.Cu") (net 2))
 (segment (start 139.5954 102.813) (end 139.5984 102.813) (width 0.3048) (layer "F.Cu") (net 2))
 (segment (start 148.8948 104.1084) (end 148.8948 104.102) (width 0.3048) (layer "F.Cu") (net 2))
 (segment (start 141.1224 125.038) (end 125.5522 125.038) (width 0.5) (layer "F.Cu") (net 2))
 (segment (start 142.4624 123.698) (end 141.1224 125.038) (width 0.5) (layer "F.Cu") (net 2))
 (segment (start 147.701978 102.502) (end 146.05 100.850022) (width 0.5) (layer "F.Cu") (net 2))
 (segment (start 125.4506 111.5252) (end 125.5014 111.5252) (width 0.3048) (layer "F.Cu") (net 2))
 (segment (start 152.965 104.083) (end 154.483511 102.564489) (width 0.5) (layer "F.Cu") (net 2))
 (segment (start 161.1634 108.655) (end 159.1564 108.655) (width 0.5) (layer "F.Cu") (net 31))
 (segment (start 168.8084 119.069) (end 168.8084 110.814) (width 0.5) (layer "F.Cu") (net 31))
 (segment (start 159.1564 108.655) (end 159.1564 110.814) (width 0.5) (layer "F.Cu") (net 31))
 (segment (start 168.8084 110.814) (end 159.1564 110.814) (width 0.5) (layer "F.Cu") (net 31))
 (segment (start 141.8874 102.686) (end 142.2654 102.94) (width 0.3048) (layer "F.Cu") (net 5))
 (segment (start 141.8874 103.067) (end 141.8874 102.686) (width 0.3048) (layer "F.Cu") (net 5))
 (segment (start 141.3764 103.067) (end 141.8874 103.067) (width 0.3048) (layer "F.Cu") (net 5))
 (segment (start 141.3764 106.725) (end 141.3764 103.067) (width 0.3048) (layer "F.Cu") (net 5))
 (segment (start 171.3484 123.768) (end 171.2784 123.698) (width 0.3048) (layer "F.Cu") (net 30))
 (segment (start 171.2784 123.698) (end 154.308 123.698) (width 0.5) (layer "F.Cu") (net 30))
 (segment (start 171.3484 108.655) (end 171.3484 123.768) (width 0.5) (layer "F.Cu") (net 30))
 (segment (start 171.3484 108.655) (end 164.0074 108.655) (width 0.5) (layer "F.Cu") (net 30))
 (segment (start 128.8064 84.9568) (end 147.2184 84.9568) (width 0.5) (layer "F.Cu") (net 7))
 (segment (start 147.2184 84.9568) (end 147.2184 88.462) (width 0.5) (layer "F.Cu") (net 7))
 (segment (start 128.8064 84.9568) (end 128.8064 88.716) (width 0.5) (layer "F.Cu") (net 7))
 (segment (start 126.0064 94.4056) (end 126.0064 90.875) (width 0.5) (layer "F.Cu") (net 28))
 (segment (start 126.2604 94.4056) (end 126.0064 94.4056) (width 0.3048) (layer "F.Cu") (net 28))
 (segment (start 122.936 97.73) (end 126.2604 94.4056) (width 0.5) (layer "F.Cu") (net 28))
 (segment (start 131.7244 90.875) (end 126.0064 90.875) (width 0.5) (layer "F.Cu") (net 28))
 (segment (start 131.7244 85.922) (end 131.7244 88.462) (width 0.5) (layer "F.Cu") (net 28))
 (segment (start 131.7244 88.462) (end 131.7244 90.875) (width 0.5) (layer "F.Cu") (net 28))
 (segment (start 122.936 100.584) (end 122.936 97.73) (width 0.5) (layer "F.Cu") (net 28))
 (segment (start 126.0064 90.875) (end 126.0064 88.716) (width 0.5) (layer "F.Cu") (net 28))
 (segment (start 122.936 107.188) (end 122.936 100.584) (width 0.5) (layer "F.Cu") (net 28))
 (segment (start 150.2604 99.2824) (end 150.2664 99.2824) (width 0.3048) (layer "F.Cu") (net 29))
 (segment (start 140.208 95.25) (end 140.208 88.392) (width 0.5) (layer "F.Cu") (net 3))
 (segment (start 140.265 95.193) (end 140.208 95.25) (width 0.3048) (layer "F.Cu") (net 3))
 (segment (start 142.805 94.177) (end 142.748 94.234) (width 0.3048) (layer "F.Cu") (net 4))
 (segment (start 142.748 94.234) (end 142.748 88.392) (width 0.5) (layer "F.Cu") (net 4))
 (segment (start 151.8604 94.177) (end 142.805 94.177) (width 0.5) (layer "F.Cu") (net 4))
 (segment (start 151.8604 99.5364) (end 151.8604 94.177) (width 0.5) (layer "F.Cu") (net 4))
 (segment (start 153.4604 99.5364) (end 153.4414 99.5364) (width 0.3048) (layer "F.Cu") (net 27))
 (segment (start 155.0604 99.5364) (end 155.0924 99.5364) (width 0.3048) (layer "F.Cu") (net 25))
 (segment (start 154.912795 89.276605) (end 154.8384 89.097) (width 0.3048) (layer "F.Cu") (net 25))
 (segment (start 154.8384 89.097) (end 154.8384 88.462) (width 0.3048) (layer "F.Cu") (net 25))
 (segment (start 155.0924 89.351) (end 154.995198 89.331665) (width 0.3048) (layer "F.Cu") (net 25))
 (segment (start 155.0924 89.351) (end 155.0924 89.351) (width 0.3048) (layer "F.Cu") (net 25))
 (segment (start 154.995198 89.331665) (end 154.912795 89.276605) (width 0.3048) (layer "F.Cu") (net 25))
 (segment (start 155.0924 99.5364) (end 155.0924 89.351) (width 0.5) (layer "F.Cu") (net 25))
 (segment (start 155.8604 99.2824) (end 155.8544 99.2824) (width 0.3048) (layer "F.Cu") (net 24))
 (segment (start 157.734 94.742) (end 157.734 88.392) (width 0.5) (layer "F.Cu") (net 24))
 (segment (start 157.734 98.044) (end 157.734 94.742) (width 0.5) (layer "F.Cu") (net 24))
 (segment (start 156.4956 99.2824) (end 157.734 98.044) (width 0.5) (layer "F.Cu") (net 24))
 (segment (start 155.8604 99.2824) (end 156.4956 99.2824) (width 0.5) (layer "F.Cu") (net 24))
 (segment (start 157.48 100.902) (end 157.5054 100.902) (width 0.3048) (layer "F.Cu") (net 23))
 (segment (start 159.9184 99.003) (end 159.9184 88.462) (width 0.5) (layer "F.Cu") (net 23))
 (segment (start 160.5214 101.702) (end 162.4584 99.765) (width 0.5) (layer "F.Cu") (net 22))
 (segment (start 162.4584 99.765) (end 162.4584 88.462) (width 0.5) (layer "F.Cu") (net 22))
 (segment (start 157.226 101.702) (end 160.5214 101.702) (width 0.5) (layer "F.Cu") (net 22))
 (segment (start 152.6604 107.8676) (end 152.6794 107.8676) (width 0.3048) (layer "F.Cu") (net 14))
 (segment (start 161.1884 113.481) (end 154.2604 113.481) (width 0.5) (layer "F.Cu") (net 16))
 (segment (start 161.1884 119.069) (end 161.1884 113.481) (width 0.5) (layer "F.Cu") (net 16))
 (segment (start 163.7284 119.4295) (end 164.3508 120.0519) (width 0.3048) (layer "F.Cu") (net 17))
 (segment (start 163.6014 112.592) (end 155.0924 112.592) (width 0.5) (layer "F.Cu") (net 17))
 (segment (start 155.0924 112.592) (end 155.0924 108.655) (width 0.5) (layer "F.Cu") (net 17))
 (segment (start 163.6014 119.069) (end 163.6014 112.592) (width 0.5) (layer "F.Cu") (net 17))
 (segment (start 163.7284 119.069) (end 163.6014 119.069) (width 0.3048) (layer "F.Cu") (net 17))
 (segment (start 163.7284 119.069) (end 163.7284 119.4295) (width 0.3048) (layer "F.Cu") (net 17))
 (segment (start 155.0604 107.8676) (end 155.0924 108.655) (width 0.3048) (layer "F.Cu") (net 17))
 (segment (start 155.8604 108.1216) (end 155.8544 108.1216) (width 0.3048) (layer "F.Cu") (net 18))
 (segment (start 166.2684 119.069) (end 166.2684 111.703) (width 0.5) (layer "F.Cu") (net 18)))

